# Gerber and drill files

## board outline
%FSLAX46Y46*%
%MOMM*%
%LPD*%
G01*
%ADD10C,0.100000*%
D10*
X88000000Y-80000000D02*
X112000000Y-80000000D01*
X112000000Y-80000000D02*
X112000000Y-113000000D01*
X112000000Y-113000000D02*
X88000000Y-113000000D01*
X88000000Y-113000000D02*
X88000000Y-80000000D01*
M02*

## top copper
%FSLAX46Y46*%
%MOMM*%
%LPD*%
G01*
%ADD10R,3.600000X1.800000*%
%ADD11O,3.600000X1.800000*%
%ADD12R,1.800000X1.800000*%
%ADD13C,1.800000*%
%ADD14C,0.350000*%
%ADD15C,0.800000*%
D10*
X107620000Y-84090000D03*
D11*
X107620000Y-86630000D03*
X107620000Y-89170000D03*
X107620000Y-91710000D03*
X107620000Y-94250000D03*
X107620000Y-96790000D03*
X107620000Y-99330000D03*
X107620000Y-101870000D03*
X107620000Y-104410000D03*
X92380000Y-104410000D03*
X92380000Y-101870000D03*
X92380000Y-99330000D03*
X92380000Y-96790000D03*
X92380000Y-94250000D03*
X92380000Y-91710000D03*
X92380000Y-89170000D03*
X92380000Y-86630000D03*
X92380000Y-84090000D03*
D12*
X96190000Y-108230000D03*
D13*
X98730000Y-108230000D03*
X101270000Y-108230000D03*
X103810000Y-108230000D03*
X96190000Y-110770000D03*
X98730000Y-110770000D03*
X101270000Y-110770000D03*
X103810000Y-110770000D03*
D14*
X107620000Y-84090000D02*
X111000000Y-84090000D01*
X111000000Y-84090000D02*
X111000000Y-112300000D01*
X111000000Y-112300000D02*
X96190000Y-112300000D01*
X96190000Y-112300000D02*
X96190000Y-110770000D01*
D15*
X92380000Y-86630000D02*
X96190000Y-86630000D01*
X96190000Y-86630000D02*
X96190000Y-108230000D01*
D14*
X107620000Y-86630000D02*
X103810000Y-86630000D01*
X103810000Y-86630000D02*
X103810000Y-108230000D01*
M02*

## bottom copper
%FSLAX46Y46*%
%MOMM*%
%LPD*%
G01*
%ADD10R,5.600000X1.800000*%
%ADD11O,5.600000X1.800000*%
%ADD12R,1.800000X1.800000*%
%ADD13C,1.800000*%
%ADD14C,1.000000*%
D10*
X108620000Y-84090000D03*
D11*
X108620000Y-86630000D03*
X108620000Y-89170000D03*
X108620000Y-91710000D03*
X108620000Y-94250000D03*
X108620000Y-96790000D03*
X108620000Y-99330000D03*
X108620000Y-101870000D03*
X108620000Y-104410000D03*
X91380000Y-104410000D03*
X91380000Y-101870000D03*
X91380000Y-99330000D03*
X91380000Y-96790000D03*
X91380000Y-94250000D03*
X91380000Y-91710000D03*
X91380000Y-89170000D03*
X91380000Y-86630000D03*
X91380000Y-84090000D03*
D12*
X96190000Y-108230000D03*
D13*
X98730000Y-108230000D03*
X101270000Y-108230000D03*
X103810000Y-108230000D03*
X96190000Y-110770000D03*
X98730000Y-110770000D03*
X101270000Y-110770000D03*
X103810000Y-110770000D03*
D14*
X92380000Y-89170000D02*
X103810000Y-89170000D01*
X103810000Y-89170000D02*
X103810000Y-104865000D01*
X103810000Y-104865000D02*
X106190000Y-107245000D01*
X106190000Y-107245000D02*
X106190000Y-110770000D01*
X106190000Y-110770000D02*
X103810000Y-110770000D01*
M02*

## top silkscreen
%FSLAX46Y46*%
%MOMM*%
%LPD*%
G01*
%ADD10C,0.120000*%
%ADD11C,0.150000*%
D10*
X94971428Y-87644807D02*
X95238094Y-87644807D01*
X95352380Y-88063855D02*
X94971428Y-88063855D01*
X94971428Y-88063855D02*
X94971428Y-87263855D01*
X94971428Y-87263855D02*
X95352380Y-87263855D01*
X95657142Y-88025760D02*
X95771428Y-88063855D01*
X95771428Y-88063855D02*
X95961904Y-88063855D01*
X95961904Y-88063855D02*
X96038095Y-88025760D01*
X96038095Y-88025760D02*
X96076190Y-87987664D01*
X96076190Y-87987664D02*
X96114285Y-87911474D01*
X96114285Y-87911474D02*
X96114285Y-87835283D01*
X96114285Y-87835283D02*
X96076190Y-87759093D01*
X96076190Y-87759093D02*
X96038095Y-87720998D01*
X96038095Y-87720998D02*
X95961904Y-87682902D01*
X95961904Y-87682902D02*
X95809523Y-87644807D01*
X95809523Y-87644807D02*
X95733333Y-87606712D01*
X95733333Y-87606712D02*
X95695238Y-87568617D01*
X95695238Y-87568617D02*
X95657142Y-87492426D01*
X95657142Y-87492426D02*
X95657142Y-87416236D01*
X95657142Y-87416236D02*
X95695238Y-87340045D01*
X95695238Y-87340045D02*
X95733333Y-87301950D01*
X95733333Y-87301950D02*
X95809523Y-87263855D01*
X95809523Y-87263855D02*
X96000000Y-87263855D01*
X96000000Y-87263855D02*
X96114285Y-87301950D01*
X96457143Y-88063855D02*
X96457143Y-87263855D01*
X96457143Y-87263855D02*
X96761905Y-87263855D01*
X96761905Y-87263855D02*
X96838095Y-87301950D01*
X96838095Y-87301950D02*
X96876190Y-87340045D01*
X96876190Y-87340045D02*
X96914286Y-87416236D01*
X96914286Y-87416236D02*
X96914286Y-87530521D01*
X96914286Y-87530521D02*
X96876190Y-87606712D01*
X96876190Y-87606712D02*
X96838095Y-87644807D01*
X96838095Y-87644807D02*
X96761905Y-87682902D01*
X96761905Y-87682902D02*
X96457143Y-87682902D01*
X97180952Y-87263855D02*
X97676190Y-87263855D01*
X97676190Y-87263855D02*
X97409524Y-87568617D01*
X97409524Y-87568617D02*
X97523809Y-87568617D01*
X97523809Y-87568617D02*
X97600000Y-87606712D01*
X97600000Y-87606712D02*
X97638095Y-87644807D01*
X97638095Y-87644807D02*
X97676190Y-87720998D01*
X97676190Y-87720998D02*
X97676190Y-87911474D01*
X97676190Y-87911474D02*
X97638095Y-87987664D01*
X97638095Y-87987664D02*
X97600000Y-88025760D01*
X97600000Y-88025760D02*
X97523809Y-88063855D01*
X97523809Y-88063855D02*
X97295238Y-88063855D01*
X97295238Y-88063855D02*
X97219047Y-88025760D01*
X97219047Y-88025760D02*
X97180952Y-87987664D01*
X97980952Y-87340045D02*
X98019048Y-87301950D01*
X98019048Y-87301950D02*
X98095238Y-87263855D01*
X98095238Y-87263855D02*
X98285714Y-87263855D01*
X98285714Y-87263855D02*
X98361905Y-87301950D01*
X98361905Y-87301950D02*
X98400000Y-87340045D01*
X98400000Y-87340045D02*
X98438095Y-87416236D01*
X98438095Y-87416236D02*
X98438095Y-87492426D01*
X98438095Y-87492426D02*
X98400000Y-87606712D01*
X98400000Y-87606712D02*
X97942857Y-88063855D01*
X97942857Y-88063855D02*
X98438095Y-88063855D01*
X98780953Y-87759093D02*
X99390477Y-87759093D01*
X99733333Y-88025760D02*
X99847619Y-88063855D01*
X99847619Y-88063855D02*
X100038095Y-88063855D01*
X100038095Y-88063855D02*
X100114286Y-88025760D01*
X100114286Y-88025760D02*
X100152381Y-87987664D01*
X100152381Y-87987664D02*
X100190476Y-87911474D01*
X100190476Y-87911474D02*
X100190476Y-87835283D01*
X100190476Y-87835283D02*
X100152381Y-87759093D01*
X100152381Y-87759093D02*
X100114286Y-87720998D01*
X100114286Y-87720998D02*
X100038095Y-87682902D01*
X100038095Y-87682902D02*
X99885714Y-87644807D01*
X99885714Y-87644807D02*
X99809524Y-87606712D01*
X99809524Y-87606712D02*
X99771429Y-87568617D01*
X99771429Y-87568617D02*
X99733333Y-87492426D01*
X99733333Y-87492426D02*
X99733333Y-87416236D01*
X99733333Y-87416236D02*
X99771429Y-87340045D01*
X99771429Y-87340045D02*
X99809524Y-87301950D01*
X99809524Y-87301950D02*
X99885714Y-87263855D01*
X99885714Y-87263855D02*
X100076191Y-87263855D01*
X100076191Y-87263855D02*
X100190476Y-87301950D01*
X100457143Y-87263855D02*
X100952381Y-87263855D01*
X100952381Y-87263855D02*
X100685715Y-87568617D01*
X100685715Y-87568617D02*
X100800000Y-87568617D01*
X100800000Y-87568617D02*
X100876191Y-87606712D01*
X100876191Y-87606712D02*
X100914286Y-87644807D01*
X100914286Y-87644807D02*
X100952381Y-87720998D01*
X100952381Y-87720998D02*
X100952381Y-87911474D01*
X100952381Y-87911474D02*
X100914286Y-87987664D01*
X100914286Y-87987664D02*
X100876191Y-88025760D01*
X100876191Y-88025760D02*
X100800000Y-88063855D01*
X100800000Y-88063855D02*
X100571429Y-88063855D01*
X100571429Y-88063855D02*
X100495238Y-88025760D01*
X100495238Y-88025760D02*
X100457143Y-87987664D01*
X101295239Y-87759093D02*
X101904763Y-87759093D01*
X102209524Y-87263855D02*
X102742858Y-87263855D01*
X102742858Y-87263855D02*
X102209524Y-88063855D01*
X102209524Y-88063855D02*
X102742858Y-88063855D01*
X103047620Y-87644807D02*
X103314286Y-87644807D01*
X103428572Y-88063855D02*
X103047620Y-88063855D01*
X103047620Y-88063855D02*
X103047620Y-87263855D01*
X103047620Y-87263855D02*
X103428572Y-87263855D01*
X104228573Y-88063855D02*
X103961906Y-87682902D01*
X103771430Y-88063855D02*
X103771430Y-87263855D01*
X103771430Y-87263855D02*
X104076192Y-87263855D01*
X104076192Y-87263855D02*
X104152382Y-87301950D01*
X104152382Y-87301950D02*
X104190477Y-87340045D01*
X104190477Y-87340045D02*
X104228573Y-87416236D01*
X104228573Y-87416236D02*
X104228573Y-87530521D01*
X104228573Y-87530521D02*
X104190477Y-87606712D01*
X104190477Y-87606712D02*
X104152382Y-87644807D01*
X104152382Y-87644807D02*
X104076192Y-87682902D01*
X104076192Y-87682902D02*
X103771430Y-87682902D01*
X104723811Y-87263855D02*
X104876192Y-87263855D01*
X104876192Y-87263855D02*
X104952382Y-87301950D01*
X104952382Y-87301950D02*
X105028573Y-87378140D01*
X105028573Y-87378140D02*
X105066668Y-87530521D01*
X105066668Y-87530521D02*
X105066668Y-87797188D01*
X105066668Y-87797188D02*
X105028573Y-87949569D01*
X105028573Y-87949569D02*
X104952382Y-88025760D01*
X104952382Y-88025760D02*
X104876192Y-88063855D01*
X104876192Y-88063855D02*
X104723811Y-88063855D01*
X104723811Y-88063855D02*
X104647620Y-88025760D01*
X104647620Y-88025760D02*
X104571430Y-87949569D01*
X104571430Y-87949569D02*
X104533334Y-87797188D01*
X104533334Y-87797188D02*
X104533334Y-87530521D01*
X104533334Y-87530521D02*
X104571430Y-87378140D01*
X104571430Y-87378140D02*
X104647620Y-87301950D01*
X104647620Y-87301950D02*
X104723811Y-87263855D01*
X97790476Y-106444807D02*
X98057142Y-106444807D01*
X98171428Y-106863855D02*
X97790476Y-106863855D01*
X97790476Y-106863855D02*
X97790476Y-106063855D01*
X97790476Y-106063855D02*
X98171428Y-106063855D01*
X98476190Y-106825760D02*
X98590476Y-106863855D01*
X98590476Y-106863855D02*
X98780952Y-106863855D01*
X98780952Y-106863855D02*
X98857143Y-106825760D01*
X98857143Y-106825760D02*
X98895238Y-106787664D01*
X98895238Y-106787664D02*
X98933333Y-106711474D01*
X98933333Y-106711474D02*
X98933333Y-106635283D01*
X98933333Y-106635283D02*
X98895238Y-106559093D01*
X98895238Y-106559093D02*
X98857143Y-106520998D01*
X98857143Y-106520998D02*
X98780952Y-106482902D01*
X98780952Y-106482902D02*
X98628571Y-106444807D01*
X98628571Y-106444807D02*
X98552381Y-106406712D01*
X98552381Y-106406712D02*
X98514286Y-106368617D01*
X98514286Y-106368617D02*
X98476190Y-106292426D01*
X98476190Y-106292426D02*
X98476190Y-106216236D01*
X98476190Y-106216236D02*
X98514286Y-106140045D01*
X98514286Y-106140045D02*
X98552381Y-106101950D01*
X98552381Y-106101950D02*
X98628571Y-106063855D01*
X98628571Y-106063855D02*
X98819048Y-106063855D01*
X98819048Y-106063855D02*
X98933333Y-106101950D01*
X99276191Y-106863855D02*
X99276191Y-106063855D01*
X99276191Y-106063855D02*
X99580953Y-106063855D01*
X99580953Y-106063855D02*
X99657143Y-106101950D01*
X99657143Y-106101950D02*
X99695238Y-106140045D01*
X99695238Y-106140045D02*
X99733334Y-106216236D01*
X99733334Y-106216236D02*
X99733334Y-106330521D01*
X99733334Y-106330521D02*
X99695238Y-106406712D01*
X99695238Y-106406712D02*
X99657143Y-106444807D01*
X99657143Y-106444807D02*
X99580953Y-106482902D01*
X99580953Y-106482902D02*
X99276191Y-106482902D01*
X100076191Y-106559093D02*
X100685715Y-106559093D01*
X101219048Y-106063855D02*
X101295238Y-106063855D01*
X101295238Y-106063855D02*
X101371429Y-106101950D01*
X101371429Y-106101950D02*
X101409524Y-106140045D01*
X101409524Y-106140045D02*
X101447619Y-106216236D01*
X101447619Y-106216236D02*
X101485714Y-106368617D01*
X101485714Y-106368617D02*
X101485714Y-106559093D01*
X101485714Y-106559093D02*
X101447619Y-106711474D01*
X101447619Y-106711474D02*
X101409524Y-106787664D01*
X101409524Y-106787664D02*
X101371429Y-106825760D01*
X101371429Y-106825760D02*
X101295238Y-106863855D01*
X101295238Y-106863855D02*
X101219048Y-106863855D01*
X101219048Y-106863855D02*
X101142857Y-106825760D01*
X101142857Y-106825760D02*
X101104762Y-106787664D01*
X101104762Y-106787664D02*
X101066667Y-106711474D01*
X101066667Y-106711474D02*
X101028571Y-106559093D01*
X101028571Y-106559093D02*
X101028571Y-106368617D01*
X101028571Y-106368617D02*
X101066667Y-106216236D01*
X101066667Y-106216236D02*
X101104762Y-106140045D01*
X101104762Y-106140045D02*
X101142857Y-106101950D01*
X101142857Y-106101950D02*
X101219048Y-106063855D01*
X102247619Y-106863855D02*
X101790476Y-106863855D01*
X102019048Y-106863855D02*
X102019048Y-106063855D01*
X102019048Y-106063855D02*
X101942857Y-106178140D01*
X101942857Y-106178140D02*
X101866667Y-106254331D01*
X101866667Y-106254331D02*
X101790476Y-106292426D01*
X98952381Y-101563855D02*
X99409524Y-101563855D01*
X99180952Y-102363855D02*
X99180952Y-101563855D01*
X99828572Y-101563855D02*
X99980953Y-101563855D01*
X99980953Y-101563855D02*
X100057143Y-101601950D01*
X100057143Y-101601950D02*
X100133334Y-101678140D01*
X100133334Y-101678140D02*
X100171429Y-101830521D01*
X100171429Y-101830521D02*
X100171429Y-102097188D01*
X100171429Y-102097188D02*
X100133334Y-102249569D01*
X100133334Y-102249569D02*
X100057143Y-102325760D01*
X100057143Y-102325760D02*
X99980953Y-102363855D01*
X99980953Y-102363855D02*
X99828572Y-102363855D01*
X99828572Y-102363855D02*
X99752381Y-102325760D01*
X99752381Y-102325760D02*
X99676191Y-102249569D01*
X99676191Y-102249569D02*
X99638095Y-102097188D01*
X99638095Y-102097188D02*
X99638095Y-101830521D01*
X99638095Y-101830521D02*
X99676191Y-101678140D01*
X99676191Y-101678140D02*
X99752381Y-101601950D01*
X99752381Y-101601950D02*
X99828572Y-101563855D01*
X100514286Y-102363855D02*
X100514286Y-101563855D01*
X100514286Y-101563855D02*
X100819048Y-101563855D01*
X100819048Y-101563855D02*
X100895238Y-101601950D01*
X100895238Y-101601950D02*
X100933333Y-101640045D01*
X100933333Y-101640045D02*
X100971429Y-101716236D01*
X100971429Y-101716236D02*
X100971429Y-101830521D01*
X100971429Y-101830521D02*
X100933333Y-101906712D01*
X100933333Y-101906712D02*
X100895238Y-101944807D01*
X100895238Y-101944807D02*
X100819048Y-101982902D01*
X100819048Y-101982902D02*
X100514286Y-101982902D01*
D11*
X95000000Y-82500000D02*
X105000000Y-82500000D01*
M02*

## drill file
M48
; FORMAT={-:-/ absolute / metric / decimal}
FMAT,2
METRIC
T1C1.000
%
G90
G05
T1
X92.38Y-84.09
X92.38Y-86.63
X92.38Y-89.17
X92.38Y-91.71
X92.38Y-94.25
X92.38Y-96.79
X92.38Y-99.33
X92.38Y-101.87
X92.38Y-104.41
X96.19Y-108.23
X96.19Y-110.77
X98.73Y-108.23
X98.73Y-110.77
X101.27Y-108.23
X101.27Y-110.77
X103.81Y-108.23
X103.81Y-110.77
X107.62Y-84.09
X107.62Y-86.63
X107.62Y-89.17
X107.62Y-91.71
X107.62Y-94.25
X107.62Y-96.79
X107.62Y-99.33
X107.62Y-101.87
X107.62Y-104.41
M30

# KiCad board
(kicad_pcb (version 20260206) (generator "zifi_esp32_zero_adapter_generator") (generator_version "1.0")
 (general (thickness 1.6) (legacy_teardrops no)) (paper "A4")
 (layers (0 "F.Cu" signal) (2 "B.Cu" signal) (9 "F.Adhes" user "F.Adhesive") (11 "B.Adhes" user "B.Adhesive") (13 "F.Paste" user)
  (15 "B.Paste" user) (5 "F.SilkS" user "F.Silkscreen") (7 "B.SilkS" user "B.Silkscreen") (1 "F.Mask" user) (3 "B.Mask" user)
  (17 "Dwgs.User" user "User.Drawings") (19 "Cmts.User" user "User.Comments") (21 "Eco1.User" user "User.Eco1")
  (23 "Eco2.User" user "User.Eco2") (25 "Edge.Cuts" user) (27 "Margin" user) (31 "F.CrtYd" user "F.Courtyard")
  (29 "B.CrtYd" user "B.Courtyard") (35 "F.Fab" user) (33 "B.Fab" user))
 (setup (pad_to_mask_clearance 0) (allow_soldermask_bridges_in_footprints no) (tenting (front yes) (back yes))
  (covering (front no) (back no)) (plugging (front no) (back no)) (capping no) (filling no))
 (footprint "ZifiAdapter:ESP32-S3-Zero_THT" (layer "F.Cu") (at 100 94.25 0)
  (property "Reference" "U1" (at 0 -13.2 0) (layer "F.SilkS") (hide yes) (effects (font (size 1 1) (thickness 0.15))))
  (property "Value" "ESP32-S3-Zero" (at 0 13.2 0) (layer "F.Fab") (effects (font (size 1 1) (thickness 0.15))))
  (fp_line (start -5 -11.75) (end 5 -11.75) (stroke (width 0.15) (type solid)) (layer "F.SilkS"))
  (pad "1" thru_hole rect (at 7.62 -10.16) (size 3.6 1.8) (drill 1) (layers "*.Cu" "*.Mask") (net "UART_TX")
   (padstack (mode front_inner_back)
    (layer "Inner" (shape rect) (size 3.6 1.8) (zone_connect -1))
    (layer "B.Cu" (shape rect) (size 5.6 1.8) (offset 1 0) (zone_connect -1))))
  (pad "2" thru_hole oval (at 7.62 -7.62) (size 3.6 1.8) (drill 1) (layers "*.Cu" "*.Mask") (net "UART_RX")
   (padstack (mode front_inner_back)
    (layer "Inner" (shape oval) (size 3.6 1.8) (zone_connect -1))
    (layer "B.Cu" (shape oval) (size 5.6 1.8) (offset 1 0) (zone_connect -1))))
  (pad "3" thru_hole oval (at 7.62 -5.08) (size 3.6 1.8) (drill 1) (layers "*.Cu" "*.Mask")
   (padstack (mode front_inner_back)
    (layer "Inner" (shape oval) (size 3.6 1.8) (zone_connect -1))
    (layer "B.Cu" (shape oval) (size 5.6 1.8) (offset 1 0) (zone_connect -1))))
  (pad "4" thru_hole oval (at 7.62 -2.54) (size 3.6 1.8) (drill 1) (layers "*.Cu" "*.Mask")
   (padstack (mode front_inner_back)
    (layer "Inner" (shape oval) (size 3.6 1.8) (zone_connect -1))
    (layer "B.Cu" (shape oval) (size 5.6 1.8) (offset 1 0) (zone_connect -1))))
  (pad "5" thru_hole oval (at 7.62 0) (size 3.6 1.8) (drill 1) (layers "*.Cu" "*.Mask")
   (padstack (mode front_inner_back)
    (layer "Inner" (shape oval) (size 3.6 1.8) (zone_connect -1))
    (layer "B.Cu" (shape oval) (size 5.6 1.8) (offset 1 0) (zone_connect -1))))
  (pad "6" thru_hole oval (at 7.62 2.54) (size 3.6 1.8) (drill 1) (layers "*.Cu" "*.Mask")
   (padstack (mode front_inner_back)
    (layer "Inner" (shape oval) (size 3.6 1.8) (zone_connect -1))
    (layer "B.Cu" (shape oval) (size 5.6 1.8) (offset 1 0) (zone_connect -1))))
  (pad "7" thru_hole oval (at 7.62 5.08) (size 3.6 1.8) (drill 1) (layers "*.Cu" "*.Mask")
   (padstack (mode front_inner_back)
    (layer "Inner" (shape oval) (size 3.6 1.8) (zone_connect -1))
    (layer "B.Cu" (shape oval) (size 5.6 1.8) (offset 1 0) (zone_connect -1))))
  (pad "8" thru_hole oval (at 7.62 7.62) (size 3.6 1.8) (drill 1) (layers "*.Cu" "*.Mask")
   (padstack (mode front_inner_back)
    (layer "Inner" (shape oval) (size 3.6 1.8) (zone_connect -1))
    (layer "B.Cu" (shape oval) (size 5.6 1.8) (offset 1 0) (zone_connect -1))))
  (pad "9" thru_hole oval (at 7.62 10.16) (size 3.6 1.8) (drill 1) (layers "*.Cu" "*.Mask")
   (padstack (mode front_inner_back)
    (layer "Inner" (shape oval) (size 3.6 1.8) (zone_connect -1))
    (layer "B.Cu" (shape oval) (size 5.6 1.8) (offset 1 0) (zone_connect -1))))
  (pad "10" thru_hole oval (at -7.62 10.16) (size 3.6 1.8) (drill 1) (layers "*.Cu" "*.Mask")
   (padstack (mode front_inner_back)
    (layer "Inner" (shape oval) (size 3.6 1.8) (zone_connect -1))
    (layer "B.Cu" (shape oval) (size 5.6 1.8) (offset -1 0) (zone_connect -1))))
  (pad "11" thru_hole oval (at -7.62 7.62) (size 3.6 1.8) (drill 1) (layers "*.Cu" "*.Mask")
   (padstack (mode front_inner_back)
    (layer "Inner" (shape oval) (size 3.6 1.8) (zone_connect -1))
    (layer "B.Cu" (shape oval) (size 5.6 1.8) (offset -1 0) (zone_connect -1))))
  (pad "12" thru_hole oval (at -7.62 5.08) (size 3.6 1.8) (drill 1) (layers "*.Cu" "*.Mask")
   (padstack (mode front_inner_back)
    (layer "Inner" (shape oval) (size 3.6 1.8) (zone_connect -1))
    (layer "B.Cu" (shape oval) (size 5.6 1.8) (offset -1 0) (zone_connect -1))))
  (pad "13" thru_hole oval (at -7.62 2.54) (size 3.6 1.8) (drill 1) (layers "*.Cu" "*.Mask")
   (padstack (mode front_inner_back)
    (layer "Inner" (shape oval) (size 3.6 1.8) (zone_connect -1))
    (layer "B.Cu" (shape oval) (size 5.6 1.8) (offset -1 0) (zone_connect -1))))
  (pad "14" thru_hole oval (at -7.62 0) (size 3.6 1.8) (drill 1) (layers "*.Cu" "*.Mask")
   (padstack (mode front_inner_back)
    (layer "Inner" (shape oval) (size 3.6 1.8) (zone_connect -1))
    (layer "B.Cu" (shape oval) (size 5.6 1.8) (offset -1 0) (zone_connect -1))))
  (pad "15" thru_hole oval (at -7.62 -2.54) (size 3.6 1.8) (drill 1) (layers "*.Cu" "*.Mask")
   (padstack (mode front_inner_back)
    (layer "Inner" (shape oval) (size 3.6 1.8) (zone_connect -1))
    (layer "B.Cu" (shape oval) (size 5.6 1.8) (offset -1 0) (zone_connect -1))))
  (pad "16" thru_hole oval (at -7.62 -5.08) (size 3.6 1.8) (drill 1) (layers "*.Cu" "*.Mask") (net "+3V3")
   (padstack (mode front_inner_back)
    (layer "Inner" (shape oval) (size 3.6 1.8) (zone_connect -1))
    (layer "B.Cu" (shape oval) (size 5.6 1.8) (offset -1 0) (zone_connect -1))))
  (pad "17" thru_hole oval (at -7.62 -7.62) (size 3.6 1.8) (drill 1) (layers "*.Cu" "*.Mask") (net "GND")
   (padstack (mode front_inner_back)
    (layer "Inner" (shape oval) (size 3.6 1.8) (zone_connect -1))
    (layer "B.Cu" (shape oval) (size 5.6 1.8) (offset -1 0) (zone_connect -1))))
  (pad "18" thru_hole oval (at -7.62 -10.16) (size 3.6 1.8) (drill 1) (layers "*.Cu" "*.Mask")
   (padstack (mode front_inner_back)
    (layer "Inner" (shape oval) (size 3.6 1.8) (zone_connect -1))
    (layer "B.Cu" (shape oval) (size 5.6 1.8) (offset -1 0) (zone_connect -1)))))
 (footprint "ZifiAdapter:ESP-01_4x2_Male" (layer "B.Cu") (at 100 109.5 0)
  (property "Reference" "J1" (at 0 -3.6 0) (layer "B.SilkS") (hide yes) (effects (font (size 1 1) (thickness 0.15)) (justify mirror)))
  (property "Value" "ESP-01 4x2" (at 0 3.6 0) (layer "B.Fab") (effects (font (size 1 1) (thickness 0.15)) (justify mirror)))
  (pad "1" thru_hole rect (at -3.81 -1.27) (size 1.8 1.8) (drill 1) (layers "*.Cu" "*.Mask") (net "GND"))
  (pad "2" thru_hole circle (at -1.27 -1.27) (size 1.8 1.8) (drill 1) (layers "*.Cu" "*.Mask"))
  (pad "3" thru_hole circle (at 1.27 -1.27) (size 1.8 1.8) (drill 1) (layers "*.Cu" "*.Mask"))
  (pad "4" thru_hole circle (at 3.81 -1.27) (size 1.8 1.8) (drill 1) (layers "*.Cu" "*.Mask") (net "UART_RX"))
  (pad "5" thru_hole circle (at -3.81 1.27) (size 1.8 1.8) (drill 1) (layers "*.Cu" "*.Mask") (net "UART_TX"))
  (pad "6" thru_hole circle (at -1.27 1.27) (size 1.8 1.8) (drill 1) (layers "*.Cu" "*.Mask"))
  (pad "7" thru_hole circle (at 1.27 1.27) (size 1.8 1.8) (drill 1) (layers "*.Cu" "*.Mask"))
  (pad "8" thru_hole circle (at 3.81 1.27) (size 1.8 1.8) (drill 1) (layers "*.Cu" "*.Mask") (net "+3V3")))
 (gr_line (start 88 80) (end 112 80) (stroke (width 0.1) (type solid)) (layer "Edge.Cuts"))
 (gr_line (start 112 80) (end 112 113) (stroke (width 0.1) (type solid)) (layer "Edge.Cuts"))
 (gr_line (start 112 113) (end 88 113) (stroke (width 0.1) (type solid)) (layer "Edge.Cuts"))
 (gr_line (start 88 113) (end 88 80) (stroke (width 0.1) (type solid)) (layer "Edge.Cuts"))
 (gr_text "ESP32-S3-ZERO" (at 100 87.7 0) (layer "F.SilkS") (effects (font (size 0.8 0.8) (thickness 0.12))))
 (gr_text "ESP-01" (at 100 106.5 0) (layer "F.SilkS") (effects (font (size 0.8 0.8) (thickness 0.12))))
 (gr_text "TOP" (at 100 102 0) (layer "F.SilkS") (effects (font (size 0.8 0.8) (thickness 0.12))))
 (segment (start 107.62 84.09) (end 111 84.09) (width 0.35) (locked yes) (layer "F.Cu") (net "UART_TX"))
 (segment (start 111 84.09) (end 111 112.3) (width 0.35) (locked yes) (layer "F.Cu") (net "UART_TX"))
 (segment (start 111 112.3) (end 96.19 112.3) (width 0.35) (locked yes) (layer "F.Cu") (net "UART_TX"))
 (segment (start 96.19 112.3) (end 96.19 110.77) (width 0.35) (locked yes) (layer "F.Cu") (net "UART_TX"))
 (segment (start 92.38 86.63) (end 96.19 86.63) (width 0.8) (locked yes) (layer "F.Cu") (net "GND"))
 (segment (start 96.19 86.63) (end 96.19 108.23) (width 0.8) (locked yes) (layer "F.Cu") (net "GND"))
 (segment (start 107.62 86.63) (end 103.81 86.63) (width 0.35) (locked yes) (layer "F.Cu") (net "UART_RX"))
 (segment (start 103.81 86.63) (end 103.81 108.23) (width 0.35) (locked yes) (layer "F.Cu") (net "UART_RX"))
 (segment (start 92.38 89.17) (end 103.81 89.17) (width 1) (locked yes) (layer "B.Cu") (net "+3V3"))
 (segment (start 103.81 89.17) (end 103.81 104.865) (width 1) (locked yes) (layer "B.Cu") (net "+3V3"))
 (segment (start 103.81 104.865) (end 106.19 107.245) (width 1) (locked yes) (layer "B.Cu") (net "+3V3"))
 (segment (start 106.19 107.245) (end 106.19 110.77) (width 1) (locked yes) (layer "B.Cu") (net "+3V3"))
 (segment (start 106.19 110.77) (end 103.81 110.77) (width 1) (locked yes) (layer "B.Cu") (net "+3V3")))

